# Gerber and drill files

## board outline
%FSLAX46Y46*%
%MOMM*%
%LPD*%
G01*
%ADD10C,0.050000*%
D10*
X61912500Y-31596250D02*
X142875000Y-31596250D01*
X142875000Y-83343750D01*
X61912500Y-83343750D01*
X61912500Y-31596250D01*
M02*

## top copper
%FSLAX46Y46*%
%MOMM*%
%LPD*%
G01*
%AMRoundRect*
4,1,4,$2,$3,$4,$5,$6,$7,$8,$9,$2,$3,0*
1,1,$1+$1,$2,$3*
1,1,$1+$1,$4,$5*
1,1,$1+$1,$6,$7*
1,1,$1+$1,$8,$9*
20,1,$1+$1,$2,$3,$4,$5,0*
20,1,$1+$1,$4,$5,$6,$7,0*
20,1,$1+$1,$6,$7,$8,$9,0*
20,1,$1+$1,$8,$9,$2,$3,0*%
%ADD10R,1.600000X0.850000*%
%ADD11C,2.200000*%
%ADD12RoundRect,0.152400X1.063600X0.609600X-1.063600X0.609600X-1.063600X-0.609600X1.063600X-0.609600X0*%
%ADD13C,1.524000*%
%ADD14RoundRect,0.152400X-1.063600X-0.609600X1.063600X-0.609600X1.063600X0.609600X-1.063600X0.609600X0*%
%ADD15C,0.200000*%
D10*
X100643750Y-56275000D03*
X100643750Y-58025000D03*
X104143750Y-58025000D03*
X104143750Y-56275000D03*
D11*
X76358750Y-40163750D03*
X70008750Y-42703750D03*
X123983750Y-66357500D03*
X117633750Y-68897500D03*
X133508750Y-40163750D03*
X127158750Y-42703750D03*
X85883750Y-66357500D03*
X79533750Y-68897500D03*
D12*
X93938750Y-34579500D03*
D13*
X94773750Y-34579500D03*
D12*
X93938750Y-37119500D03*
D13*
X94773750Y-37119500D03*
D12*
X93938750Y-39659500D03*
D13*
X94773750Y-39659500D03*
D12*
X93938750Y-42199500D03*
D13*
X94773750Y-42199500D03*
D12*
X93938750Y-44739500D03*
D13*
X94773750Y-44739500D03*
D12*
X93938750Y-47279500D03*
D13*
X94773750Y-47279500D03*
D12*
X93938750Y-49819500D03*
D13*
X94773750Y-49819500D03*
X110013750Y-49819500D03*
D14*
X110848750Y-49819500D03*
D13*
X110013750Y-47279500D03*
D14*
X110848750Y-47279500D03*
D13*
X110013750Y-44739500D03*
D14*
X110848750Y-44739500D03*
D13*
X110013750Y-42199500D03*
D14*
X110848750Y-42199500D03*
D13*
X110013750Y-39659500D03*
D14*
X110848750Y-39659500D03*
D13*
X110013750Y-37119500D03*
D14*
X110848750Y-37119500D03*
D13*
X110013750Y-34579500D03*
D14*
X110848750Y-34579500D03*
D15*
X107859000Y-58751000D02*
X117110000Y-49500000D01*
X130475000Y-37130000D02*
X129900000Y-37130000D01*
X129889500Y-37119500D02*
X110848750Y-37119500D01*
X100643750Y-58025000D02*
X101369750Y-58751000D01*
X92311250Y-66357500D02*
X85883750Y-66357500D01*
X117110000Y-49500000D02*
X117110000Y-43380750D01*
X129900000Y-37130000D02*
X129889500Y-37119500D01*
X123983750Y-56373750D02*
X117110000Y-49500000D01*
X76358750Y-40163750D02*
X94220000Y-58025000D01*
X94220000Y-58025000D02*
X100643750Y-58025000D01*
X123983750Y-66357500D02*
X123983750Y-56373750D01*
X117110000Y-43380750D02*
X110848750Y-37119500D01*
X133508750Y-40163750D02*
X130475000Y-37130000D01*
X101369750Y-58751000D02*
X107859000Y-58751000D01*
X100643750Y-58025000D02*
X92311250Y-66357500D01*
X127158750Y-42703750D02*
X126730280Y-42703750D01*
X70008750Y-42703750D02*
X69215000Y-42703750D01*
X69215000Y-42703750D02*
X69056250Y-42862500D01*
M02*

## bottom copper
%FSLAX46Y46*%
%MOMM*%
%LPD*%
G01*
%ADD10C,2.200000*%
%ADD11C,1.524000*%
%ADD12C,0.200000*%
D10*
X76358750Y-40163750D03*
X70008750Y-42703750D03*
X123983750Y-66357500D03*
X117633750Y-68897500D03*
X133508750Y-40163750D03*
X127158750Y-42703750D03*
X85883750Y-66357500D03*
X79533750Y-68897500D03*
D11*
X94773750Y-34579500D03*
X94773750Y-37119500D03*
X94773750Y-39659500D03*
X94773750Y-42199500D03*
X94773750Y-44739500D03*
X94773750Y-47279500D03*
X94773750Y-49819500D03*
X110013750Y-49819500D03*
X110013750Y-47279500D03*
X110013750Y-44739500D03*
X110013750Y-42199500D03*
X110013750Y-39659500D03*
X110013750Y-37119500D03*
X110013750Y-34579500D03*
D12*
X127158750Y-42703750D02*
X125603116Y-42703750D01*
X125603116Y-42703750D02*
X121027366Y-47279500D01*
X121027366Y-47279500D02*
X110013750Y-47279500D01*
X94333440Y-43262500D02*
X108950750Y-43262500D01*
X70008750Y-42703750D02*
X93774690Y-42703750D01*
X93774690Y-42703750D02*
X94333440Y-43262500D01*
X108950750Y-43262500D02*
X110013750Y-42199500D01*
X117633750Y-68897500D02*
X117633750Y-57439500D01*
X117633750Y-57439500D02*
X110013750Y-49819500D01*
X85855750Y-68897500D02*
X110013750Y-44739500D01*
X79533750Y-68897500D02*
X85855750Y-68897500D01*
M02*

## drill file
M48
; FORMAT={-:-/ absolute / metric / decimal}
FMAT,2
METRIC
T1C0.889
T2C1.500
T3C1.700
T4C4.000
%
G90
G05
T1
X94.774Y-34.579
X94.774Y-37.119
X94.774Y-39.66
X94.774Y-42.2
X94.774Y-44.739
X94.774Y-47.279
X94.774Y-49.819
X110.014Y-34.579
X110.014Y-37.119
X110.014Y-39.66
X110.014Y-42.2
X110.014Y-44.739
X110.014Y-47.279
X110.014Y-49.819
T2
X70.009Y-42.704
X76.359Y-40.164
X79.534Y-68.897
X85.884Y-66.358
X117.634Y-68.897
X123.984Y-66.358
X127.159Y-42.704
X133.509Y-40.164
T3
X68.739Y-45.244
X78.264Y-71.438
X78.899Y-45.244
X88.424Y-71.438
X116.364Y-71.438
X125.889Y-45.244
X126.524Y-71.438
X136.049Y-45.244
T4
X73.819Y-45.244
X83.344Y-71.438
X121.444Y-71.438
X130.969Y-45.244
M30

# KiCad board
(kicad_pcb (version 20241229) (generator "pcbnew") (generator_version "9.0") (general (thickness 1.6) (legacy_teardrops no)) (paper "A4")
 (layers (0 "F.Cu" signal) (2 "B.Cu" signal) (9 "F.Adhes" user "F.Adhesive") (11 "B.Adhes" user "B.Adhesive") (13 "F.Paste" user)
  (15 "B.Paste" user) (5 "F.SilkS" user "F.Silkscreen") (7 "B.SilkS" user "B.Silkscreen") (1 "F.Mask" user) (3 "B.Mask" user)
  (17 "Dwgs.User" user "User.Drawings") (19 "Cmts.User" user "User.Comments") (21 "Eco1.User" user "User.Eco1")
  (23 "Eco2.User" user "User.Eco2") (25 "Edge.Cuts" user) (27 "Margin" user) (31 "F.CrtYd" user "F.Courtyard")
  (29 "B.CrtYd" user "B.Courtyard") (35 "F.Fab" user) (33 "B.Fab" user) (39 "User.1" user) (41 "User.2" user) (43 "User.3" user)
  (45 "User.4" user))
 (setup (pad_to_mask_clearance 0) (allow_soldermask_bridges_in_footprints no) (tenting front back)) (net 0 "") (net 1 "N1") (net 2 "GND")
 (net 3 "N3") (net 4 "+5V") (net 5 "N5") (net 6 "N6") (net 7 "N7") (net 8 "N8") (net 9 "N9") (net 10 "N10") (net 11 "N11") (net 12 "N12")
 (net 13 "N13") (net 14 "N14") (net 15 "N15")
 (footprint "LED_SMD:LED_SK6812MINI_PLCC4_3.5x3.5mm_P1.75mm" (layer "F.Cu") (at 102.39375 57.15)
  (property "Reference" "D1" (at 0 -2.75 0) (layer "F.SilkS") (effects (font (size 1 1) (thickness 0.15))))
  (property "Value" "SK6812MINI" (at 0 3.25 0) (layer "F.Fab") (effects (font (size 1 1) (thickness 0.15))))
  (pad "1" smd rect (at -1.75 -0.875) (size 1.6 0.85) (layers "F.Cu" "F.Mask" "F.Paste") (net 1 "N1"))
  (pad "2" smd rect (at -1.75 0.875) (size 1.6 0.85) (layers "F.Cu" "F.Mask" "F.Paste") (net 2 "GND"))
  (pad "3" smd rect (at 1.75 0.875) (size 1.6 0.85) (layers "F.Cu" "F.Mask" "F.Paste") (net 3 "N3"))
  (pad "4" smd rect (at 1.75 -0.875) (size 1.6 0.85) (layers "F.Cu" "F.Mask" "F.Paste") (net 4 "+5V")))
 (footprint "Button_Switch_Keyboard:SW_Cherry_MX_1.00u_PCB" (layer "F.Cu") (at 76.35875 40.16375)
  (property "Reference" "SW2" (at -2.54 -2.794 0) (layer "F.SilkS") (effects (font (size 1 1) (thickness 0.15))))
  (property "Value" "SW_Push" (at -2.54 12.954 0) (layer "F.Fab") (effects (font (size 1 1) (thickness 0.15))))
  (pad "" np_thru_hole circle (at -7.62 5.08) (size 1.7 1.7) (drill 1.7) (layers "*.Cu" "*.Mask"))
  (pad "" np_thru_hole circle (at -2.54 5.08) (size 4 4) (drill 4) (layers "*.Cu" "*.Mask"))
  (pad "" np_thru_hole circle (at 2.54 5.08) (size 1.7 1.7) (drill 1.7) (layers "*.Cu" "*.Mask"))
  (pad "1" thru_hole circle (at 0 0) (size 2.2 2.2) (drill 1.5) (layers "*.Cu" "*.Mask") (remove_unused_layers no) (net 2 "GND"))
  (pad "2" thru_hole circle (at -6.35 2.54) (size 2.2 2.2) (drill 1.5) (layers "*.Cu" "*.Mask") (remove_unused_layers no) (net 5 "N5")))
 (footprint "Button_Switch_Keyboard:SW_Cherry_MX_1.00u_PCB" (layer "F.Cu") (at 123.98375 66.3575)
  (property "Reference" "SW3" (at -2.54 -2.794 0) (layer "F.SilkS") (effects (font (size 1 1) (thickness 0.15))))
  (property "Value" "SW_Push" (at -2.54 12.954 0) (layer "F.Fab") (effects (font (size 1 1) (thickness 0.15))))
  (pad "" np_thru_hole circle (at -7.62 5.08) (size 1.7 1.7) (drill 1.7) (layers "*.Cu" "*.Mask"))
  (pad "" np_thru_hole circle (at -2.54 5.08) (size 4 4) (drill 4) (layers "*.Cu" "*.Mask"))
  (pad "" np_thru_hole circle (at 2.54 5.08) (size 1.7 1.7) (drill 1.7) (layers "*.Cu" "*.Mask"))
  (pad "1" thru_hole circle (at 0 0) (size 2.2 2.2) (drill 1.5) (layers "*.Cu" "*.Mask") (remove_unused_layers no) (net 2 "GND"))
  (pad "2" thru_hole circle (at -6.35 2.54) (size 2.2 2.2) (drill 1.5) (layers "*.Cu" "*.Mask") (remove_unused_layers no) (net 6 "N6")))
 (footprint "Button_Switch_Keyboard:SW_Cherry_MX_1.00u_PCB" (layer "F.Cu") (at 133.50875 40.16375)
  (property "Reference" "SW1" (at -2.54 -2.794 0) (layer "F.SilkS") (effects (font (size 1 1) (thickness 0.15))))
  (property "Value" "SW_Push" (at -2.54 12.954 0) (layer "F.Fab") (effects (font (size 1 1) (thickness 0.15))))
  (pad "" np_thru_hole circle (at -7.62 5.08) (size 1.7 1.7) (drill 1.7) (layers "*.Cu" "*.Mask"))
  (pad "" np_thru_hole circle (at -2.54 5.08) (size 4 4) (drill 4) (layers "*.Cu" "*.Mask"))
  (pad "" np_thru_hole circle (at 2.54 5.08) (size 1.7 1.7) (drill 1.7) (layers "*.Cu" "*.Mask"))
  (pad "1" thru_hole circle (at 0 0) (size 2.2 2.2) (drill 1.5) (layers "*.Cu" "*.Mask") (remove_unused_layers no) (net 2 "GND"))
  (pad "2" thru_hole circle (at -6.35 2.54) (size 2.2 2.2) (drill 1.5) (layers "*.Cu" "*.Mask") (remove_unused_layers no) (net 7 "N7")))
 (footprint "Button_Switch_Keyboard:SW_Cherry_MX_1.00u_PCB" (layer "F.Cu") (at 85.88375 66.3575)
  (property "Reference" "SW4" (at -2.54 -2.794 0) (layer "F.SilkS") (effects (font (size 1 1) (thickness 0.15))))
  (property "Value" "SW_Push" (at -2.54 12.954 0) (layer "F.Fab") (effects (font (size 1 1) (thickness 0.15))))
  (pad "" np_thru_hole circle (at -7.62 5.08) (size 1.7 1.7) (drill 1.7) (layers "*.Cu" "*.Mask"))
  (pad "" np_thru_hole circle (at -2.54 5.08) (size 4 4) (drill 4) (layers "*.Cu" "*.Mask"))
  (pad "" np_thru_hole circle (at 2.54 5.08) (size 1.7 1.7) (drill 1.7) (layers "*.Cu" "*.Mask"))
  (pad "1" thru_hole circle (at 0 0) (size 2.2 2.2) (drill 1.5) (layers "*.Cu" "*.Mask") (remove_unused_layers no) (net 2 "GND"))
  (pad "2" thru_hole circle (at -6.35 2.54) (size 2.2 2.2) (drill 1.5) (layers "*.Cu" "*.Mask") (remove_unused_layers no) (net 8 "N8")))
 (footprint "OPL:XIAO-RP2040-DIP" (layer "F.Cu") (at 102.39375 42.1995)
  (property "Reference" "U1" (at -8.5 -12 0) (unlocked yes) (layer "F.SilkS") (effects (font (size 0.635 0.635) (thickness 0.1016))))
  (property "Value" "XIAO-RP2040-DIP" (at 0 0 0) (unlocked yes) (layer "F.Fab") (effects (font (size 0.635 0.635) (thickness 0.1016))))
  (pad "1" smd roundrect (at -8.455 -7.62 180) (size 2.432 1.524) (layers "F.Cu" "F.Mask") (roundrect_rratio 0.1) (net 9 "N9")
   (thermal_bridge_angle 45))
  (pad "1" thru_hole circle (at -7.62 -7.62 180) (size 1.524 1.524) (drill 0.889) (layers "*.Cu" "*.Mask") (remove_unused_layers no)
   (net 9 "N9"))
  (pad "2" smd roundrect (at -8.455 -5.08 180) (size 2.432 1.524) (layers "F.Cu" "F.Mask") (roundrect_rratio 0.1) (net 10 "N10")
   (thermal_bridge_angle 45))
  (pad "2" thru_hole circle (at -7.62 -5.08 180) (size 1.524 1.524) (drill 0.889) (layers "*.Cu" "*.Mask") (remove_unused_layers no)
   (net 10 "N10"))
  (pad "3" smd roundrect (at -8.455 -2.54 180) (size 2.432 1.524) (layers "F.Cu" "F.Mask") (roundrect_rratio 0.1) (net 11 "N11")
   (thermal_bridge_angle 45))
  (pad "3" thru_hole circle (at -7.62 -2.54 180) (size 1.524 1.524) (drill 0.889) (layers "*.Cu" "*.Mask") (remove_unused_layers no)
   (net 11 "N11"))
  (pad "4" smd roundrect (at -8.455 0 180) (size 2.432 1.524) (layers "F.Cu" "F.Mask") (roundrect_rratio 0.1) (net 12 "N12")
   (thermal_bridge_angle 45))
  (pad "4" thru_hole circle (at -7.62 0 180) (size 1.524 1.524) (drill 0.889) (layers "*.Cu" "*.Mask") (remove_unused_layers no)
   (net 12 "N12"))
  (pad "5" smd roundrect (at -8.455 2.54 180) (size 2.432 1.524) (layers "F.Cu" "F.Mask") (roundrect_rratio 0.1) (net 3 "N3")
   (thermal_bridge_angle 45))
  (pad "5" thru_hole circle (at -7.62 2.54 180) (size 1.524 1.524) (drill 0.889) (layers "*.Cu" "*.Mask") (remove_unused_layers no)
   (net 3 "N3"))
  (pad "6" smd roundrect (at -8.455 5.08 180) (size 2.432 1.524) (layers "F.Cu" "F.Mask") (roundrect_rratio 0.1) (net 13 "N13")
   (thermal_bridge_angle 45))
  (pad "6" thru_hole circle (at -7.62 5.08 180) (size 1.524 1.524) (drill 0.889) (layers "*.Cu" "*.Mask") (remove_unused_layers no)
   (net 13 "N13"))
  (pad "7" smd roundrect (at -8.455 7.62 180) (size 2.432 1.524) (layers "F.Cu" "F.Mask") (roundrect_rratio 0.1) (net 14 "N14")
   (thermal_bridge_angle 45))
  (pad "7" thru_hole circle (at -7.62 7.62 180) (size 1.524 1.524) (drill 0.889) (layers "*.Cu" "*.Mask") (remove_unused_layers no)
   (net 14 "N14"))
  (pad "8" thru_hole circle (at 7.62 7.62) (size 1.524 1.524) (drill 0.889) (layers "*.Cu" "*.Mask") (remove_unused_layers no) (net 6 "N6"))
  (pad "8" smd roundrect (at 8.455 7.62) (size 2.432 1.524) (layers "F.Cu" "F.Mask") (roundrect_rratio 0.1) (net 6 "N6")
   (thermal_bridge_angle 45))
  (pad "9" thru_hole circle (at 7.62 5.08) (size 1.524 1.524) (drill 0.889) (layers "*.Cu" "*.Mask") (remove_unused_layers no) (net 7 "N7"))
  (pad "9" smd roundrect (at 8.455 5.08) (size 2.432 1.524) (layers "F.Cu" "F.Mask") (roundrect_rratio 0.1) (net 7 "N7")
   (thermal_bridge_angle 45))
  (pad "10" thru_hole circle (at 7.62 2.54) (size 1.524 1.524) (drill 0.889) (layers "*.Cu" "*.Mask") (remove_unused_layers no) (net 8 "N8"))
  (pad "10" smd roundrect (at 8.455 2.54) (size 2.432 1.524) (layers "F.Cu" "F.Mask") (roundrect_rratio 0.1) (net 8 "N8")
   (thermal_bridge_angle 45))
  (pad "11" thru_hole circle (at 7.62 0) (size 1.524 1.524) (drill 0.889) (layers "*.Cu" "*.Mask") (remove_unused_layers no) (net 5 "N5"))
  (pad "11" smd roundrect (at 8.455 0) (size 2.432 1.524) (layers "F.Cu" "F.Mask") (roundrect_rratio 0.1) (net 5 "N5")
   (thermal_bridge_angle 45))
  (pad "12" thru_hole circle (at 7.62 -2.54) (size 1.524 1.524) (drill 0.889) (layers "*.Cu" "*.Mask") (remove_unused_layers no)
   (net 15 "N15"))
  (pad "12" smd roundrect (at 8.455 -2.54) (size 2.432 1.524) (layers "F.Cu" "F.Mask") (roundrect_rratio 0.1) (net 15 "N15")
   (thermal_bridge_angle 45))
  (pad "13" thru_hole circle (at 7.62 -5.08) (size 1.524 1.524) (drill 0.889) (layers "*.Cu" "*.Mask") (remove_unused_layers no)
   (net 2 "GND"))
  (pad "13" smd roundrect (at 8.455 -5.08) (size 2.432 1.524) (layers "F.Cu" "F.Mask") (roundrect_rratio 0.1) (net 2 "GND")
   (thermal_bridge_angle 45))
  (pad "14" thru_hole circle (at 7.62 -7.62) (size 1.524 1.524) (drill 0.889) (layers "*.Cu" "*.Mask") (remove_unused_layers no)
   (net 4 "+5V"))
  (pad "14" smd roundrect (at 8.455 -7.62) (size 2.432 1.524) (layers "F.Cu" "F.Mask") (roundrect_rratio 0.1) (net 4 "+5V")
   (thermal_bridge_angle 45)))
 (gr_rect (start 61.9125 31.59625) (end 142.875 83.34375) (stroke (width 0.05) (type default)) (fill no) (layer "Edge.Cuts"))
 (segment (start 107.859 58.751) (end 117.11 49.5) (width 0.2) (layer "F.Cu") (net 2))
 (segment (start 130.475 37.13) (end 129.9 37.13) (width 0.2) (layer "F.Cu") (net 2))
 (segment (start 129.8895 37.1195) (end 110.84875 37.1195) (width 0.2) (layer "F.Cu") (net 2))
 (segment (start 100.64375 58.025) (end 101.36975 58.751) (width 0.2) (layer "F.Cu") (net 2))
 (segment (start 92.31125 66.3575) (end 85.88375 66.3575) (width 0.2) (layer "F.Cu") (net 2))
 (segment (start 117.11 49.5) (end 117.11 43.38075) (width 0.2) (layer "F.Cu") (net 2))
 (segment (start 129.9 37.13) (end 129.8895 37.1195) (width 0.2) (layer "F.Cu") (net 2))
 (segment (start 123.98375 56.37375) (end 117.11 49.5) (width 0.2) (layer "F.Cu") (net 2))
 (segment (start 76.35875 40.16375) (end 94.22 58.025) (width 0.2) (layer "F.Cu") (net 2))
 (segment (start 94.22 58.025) (end 100.64375 58.025) (width 0.2) (layer "F.Cu") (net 2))
 (segment (start 123.98375 66.3575) (end 123.98375 56.37375) (width 0.2) (layer "F.Cu") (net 2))
 (segment (start 117.11 43.38075) (end 110.84875 37.1195) (width 0.2) (layer "F.Cu") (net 2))
 (segment (start 133.50875 40.16375) (end 130.475 37.13) (width 0.2) (layer "F.Cu") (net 2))
 (segment (start 101.36975 58.751) (end 107.859 58.751) (width 0.2) (layer "F.Cu") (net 2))
 (segment (start 100.64375 58.025) (end 92.31125 66.3575) (width 0.2) (layer "F.Cu") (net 2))
 (segment (start 127.15875 42.70375) (end 126.73028 42.70375) (width 0.2) (layer "F.Cu") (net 7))
 (segment (start 127.15875 42.70375) (end 125.603116 42.70375) (width 0.2) (layer "B.Cu") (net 7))
 (segment (start 125.603116 42.70375) (end 121.027366 47.2795) (width 0.2) (layer "B.Cu") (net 7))
 (segment (start 121.027366 47.2795) (end 110.01375 47.2795) (width 0.2) (layer "B.Cu") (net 7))
 (segment (start 70.00875 42.70375) (end 69.215 42.70375) (width 0.2) (layer "F.Cu") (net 5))
 (segment (start 69.215 42.70375) (end 69.05625 42.8625) (width 0.2) (layer "F.Cu") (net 5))
 (segment (start 94.33344 43.2625) (end 108.95075 43.2625) (width 0.2) (layer "B.Cu") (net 5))
 (segment (start 70.00875 42.70375) (end 93.77469 42.70375) (width 0.2) (layer "B.Cu") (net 5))
 (segment (start 93.77469 42.70375) (end 94.33344 43.2625) (width 0.2) (layer "B.Cu") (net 5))
 (segment (start 108.95075 43.2625) (end 110.01375 42.1995) (width 0.2) (layer "B.Cu") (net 5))
 (segment (start 117.63375 68.8975) (end 117.63375 57.4395) (width 0.2) (layer "B.Cu") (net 6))
 (segment (start 117.63375 57.4395) (end 110.01375 49.8195) (width 0.2) (layer "B.Cu") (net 6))
 (segment (start 85.85575 68.8975) (end 110.01375 44.7395) (width 0.2) (layer "B.Cu") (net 8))
 (segment (start 79.53375 68.8975) (end 85.85575 68.8975) (width 0.2) (layer "B.Cu") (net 8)))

